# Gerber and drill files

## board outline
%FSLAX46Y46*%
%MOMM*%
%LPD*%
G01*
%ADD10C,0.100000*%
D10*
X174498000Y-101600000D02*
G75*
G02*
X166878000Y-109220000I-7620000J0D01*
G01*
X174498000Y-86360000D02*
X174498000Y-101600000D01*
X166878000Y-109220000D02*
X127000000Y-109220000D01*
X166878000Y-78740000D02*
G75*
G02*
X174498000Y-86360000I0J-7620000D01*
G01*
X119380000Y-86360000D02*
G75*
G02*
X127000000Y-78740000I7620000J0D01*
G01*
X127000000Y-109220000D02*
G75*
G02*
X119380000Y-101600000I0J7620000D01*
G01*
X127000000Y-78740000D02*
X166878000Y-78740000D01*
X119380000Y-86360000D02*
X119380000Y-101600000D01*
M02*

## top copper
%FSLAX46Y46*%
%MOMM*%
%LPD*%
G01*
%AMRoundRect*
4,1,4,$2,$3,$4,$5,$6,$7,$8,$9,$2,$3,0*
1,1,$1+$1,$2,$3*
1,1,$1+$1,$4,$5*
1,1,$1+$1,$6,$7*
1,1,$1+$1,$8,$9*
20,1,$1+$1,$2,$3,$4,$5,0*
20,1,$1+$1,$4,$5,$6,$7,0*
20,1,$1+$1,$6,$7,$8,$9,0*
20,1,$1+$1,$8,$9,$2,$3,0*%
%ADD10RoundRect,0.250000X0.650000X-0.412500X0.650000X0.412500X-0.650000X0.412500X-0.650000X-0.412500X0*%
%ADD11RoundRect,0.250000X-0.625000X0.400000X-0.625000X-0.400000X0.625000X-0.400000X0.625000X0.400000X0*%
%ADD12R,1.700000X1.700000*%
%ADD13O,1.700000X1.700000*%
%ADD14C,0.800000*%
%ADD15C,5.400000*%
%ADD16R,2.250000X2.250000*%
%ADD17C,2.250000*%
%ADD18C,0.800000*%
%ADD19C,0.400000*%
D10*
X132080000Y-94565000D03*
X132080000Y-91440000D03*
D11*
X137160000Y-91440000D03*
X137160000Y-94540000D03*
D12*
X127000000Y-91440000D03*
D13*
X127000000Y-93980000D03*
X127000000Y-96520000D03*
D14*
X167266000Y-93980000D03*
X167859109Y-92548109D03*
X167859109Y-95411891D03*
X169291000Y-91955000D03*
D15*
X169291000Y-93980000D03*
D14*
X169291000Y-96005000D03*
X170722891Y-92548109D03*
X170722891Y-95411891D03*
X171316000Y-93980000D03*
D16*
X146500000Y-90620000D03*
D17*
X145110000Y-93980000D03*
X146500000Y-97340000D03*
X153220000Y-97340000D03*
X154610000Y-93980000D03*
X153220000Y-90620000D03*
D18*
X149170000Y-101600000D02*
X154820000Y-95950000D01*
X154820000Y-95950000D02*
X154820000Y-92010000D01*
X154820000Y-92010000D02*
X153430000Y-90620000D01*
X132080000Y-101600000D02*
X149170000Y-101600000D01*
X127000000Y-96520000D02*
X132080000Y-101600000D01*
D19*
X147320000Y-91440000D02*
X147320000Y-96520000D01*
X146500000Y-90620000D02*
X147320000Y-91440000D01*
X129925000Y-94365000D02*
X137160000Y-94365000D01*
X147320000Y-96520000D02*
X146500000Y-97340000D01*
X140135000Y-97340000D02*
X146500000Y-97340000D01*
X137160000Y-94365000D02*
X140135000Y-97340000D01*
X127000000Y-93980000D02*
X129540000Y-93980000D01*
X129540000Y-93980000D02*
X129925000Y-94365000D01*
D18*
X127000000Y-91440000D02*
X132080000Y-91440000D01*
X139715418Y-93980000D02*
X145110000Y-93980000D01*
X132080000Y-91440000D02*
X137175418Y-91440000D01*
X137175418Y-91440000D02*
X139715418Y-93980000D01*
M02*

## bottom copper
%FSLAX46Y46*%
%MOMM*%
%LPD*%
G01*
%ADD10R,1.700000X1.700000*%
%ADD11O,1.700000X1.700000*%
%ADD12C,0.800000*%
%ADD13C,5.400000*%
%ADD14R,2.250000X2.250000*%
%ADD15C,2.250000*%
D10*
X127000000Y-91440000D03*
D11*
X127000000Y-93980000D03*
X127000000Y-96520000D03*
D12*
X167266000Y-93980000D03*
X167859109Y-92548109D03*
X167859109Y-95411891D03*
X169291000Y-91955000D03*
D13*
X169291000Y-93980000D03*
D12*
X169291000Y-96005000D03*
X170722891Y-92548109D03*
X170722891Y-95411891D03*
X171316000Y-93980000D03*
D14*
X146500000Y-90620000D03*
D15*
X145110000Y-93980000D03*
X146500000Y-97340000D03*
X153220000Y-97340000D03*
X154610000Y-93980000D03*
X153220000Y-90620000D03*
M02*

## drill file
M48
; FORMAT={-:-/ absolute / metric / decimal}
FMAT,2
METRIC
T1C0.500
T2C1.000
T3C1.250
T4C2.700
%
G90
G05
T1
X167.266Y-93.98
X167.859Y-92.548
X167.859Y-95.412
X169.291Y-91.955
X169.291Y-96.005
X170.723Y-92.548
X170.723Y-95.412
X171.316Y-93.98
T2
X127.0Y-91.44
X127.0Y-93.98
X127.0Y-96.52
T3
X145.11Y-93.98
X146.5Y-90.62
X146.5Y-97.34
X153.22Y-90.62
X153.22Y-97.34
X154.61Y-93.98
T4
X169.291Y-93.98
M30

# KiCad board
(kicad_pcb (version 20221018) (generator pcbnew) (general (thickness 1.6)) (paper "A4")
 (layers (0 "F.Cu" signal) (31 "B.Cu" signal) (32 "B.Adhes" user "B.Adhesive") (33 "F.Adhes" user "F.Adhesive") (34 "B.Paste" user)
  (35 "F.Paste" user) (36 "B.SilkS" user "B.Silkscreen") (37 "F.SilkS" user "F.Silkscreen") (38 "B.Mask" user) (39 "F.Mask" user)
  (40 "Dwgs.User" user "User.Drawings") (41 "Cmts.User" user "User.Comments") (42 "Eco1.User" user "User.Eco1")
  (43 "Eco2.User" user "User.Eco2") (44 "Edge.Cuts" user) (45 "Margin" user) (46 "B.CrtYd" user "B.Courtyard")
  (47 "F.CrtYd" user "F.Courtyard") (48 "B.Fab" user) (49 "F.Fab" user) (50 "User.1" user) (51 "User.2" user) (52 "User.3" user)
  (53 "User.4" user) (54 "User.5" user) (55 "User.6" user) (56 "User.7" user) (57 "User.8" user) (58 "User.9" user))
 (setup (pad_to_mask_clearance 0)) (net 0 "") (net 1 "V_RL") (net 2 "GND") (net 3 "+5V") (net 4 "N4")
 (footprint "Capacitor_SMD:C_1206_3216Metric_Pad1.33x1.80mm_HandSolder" (layer "F.Cu") (at 132.08 93.0025 90)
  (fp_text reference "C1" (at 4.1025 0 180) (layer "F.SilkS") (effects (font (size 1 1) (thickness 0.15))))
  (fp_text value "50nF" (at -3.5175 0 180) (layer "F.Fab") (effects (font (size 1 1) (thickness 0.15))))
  (pad "1" smd roundrect (at -1.5625 0 90) (size 1.325 1.8) (layers "F.Cu" "F.Paste" "F.Mask") (roundrect_rratio 0.1886792453)
   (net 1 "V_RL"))
  (pad "2" smd roundrect (at 1.5625 0 90) (size 1.325 1.8) (layers "F.Cu" "F.Paste" "F.Mask") (roundrect_rratio 0.1886792453) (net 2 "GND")))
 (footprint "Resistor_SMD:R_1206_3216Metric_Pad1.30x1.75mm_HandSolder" (layer "F.Cu") (at 137.16 92.99 -90)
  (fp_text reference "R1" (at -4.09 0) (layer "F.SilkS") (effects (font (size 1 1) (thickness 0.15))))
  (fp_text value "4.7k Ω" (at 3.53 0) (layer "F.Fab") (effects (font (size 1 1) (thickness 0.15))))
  (pad "1" smd roundrect (at -1.55 0 270) (size 1.3 1.75) (layers "F.Cu" "F.Paste" "F.Mask") (roundrect_rratio 0.1923076923) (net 2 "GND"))
  (pad "2" smd roundrect (at 1.55 0 270) (size 1.3 1.75) (layers "F.Cu" "F.Paste" "F.Mask") (roundrect_rratio 0.1923076923) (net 1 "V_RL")))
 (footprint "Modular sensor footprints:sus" (layer "F.Cu") (at 149.86 93.98)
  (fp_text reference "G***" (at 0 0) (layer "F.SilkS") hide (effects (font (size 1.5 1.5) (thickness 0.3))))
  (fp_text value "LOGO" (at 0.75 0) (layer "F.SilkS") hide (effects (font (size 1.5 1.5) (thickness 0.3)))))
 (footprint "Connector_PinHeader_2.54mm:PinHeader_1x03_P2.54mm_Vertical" (layer "F.Cu") (at 127 91.44)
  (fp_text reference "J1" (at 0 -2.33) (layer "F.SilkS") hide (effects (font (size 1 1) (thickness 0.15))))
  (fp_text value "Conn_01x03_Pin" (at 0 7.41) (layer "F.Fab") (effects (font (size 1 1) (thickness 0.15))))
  (pad "1" thru_hole rect (at 0 0) (size 1.7 1.7) (drill 1) (layers "*.Cu" "*.Mask") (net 2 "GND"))
  (pad "2" thru_hole oval (at 0 2.54) (size 1.7 1.7) (drill 1) (layers "*.Cu" "*.Mask") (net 1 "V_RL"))
  (pad "3" thru_hole oval (at 0 5.08) (size 1.7 1.7) (drill 1) (layers "*.Cu" "*.Mask") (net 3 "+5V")))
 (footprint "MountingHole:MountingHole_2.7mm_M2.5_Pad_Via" (layer "F.Cu") (at 169.291 93.98)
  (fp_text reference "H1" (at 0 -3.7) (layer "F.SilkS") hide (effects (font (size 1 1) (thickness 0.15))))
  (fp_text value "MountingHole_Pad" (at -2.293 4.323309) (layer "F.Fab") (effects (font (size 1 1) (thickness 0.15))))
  (pad "1" thru_hole circle (at -2.025 0) (size 0.8 0.8) (drill 0.5) (layers "*.Cu" "*.Mask") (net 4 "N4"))
  (pad "1" thru_hole circle (at -1.431891 -1.431891) (size 0.8 0.8) (drill 0.5) (layers "*.Cu" "*.Mask") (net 4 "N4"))
  (pad "1" thru_hole circle (at -1.431891 1.431891) (size 0.8 0.8) (drill 0.5) (layers "*.Cu" "*.Mask") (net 4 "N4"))
  (pad "1" thru_hole circle (at 0 -2.025) (size 0.8 0.8) (drill 0.5) (layers "*.Cu" "*.Mask") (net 4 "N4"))
  (pad "1" thru_hole circle (at 0 0) (size 5.4 5.4) (drill 2.7) (layers "*.Cu" "*.Mask") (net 4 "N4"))
  (pad "1" thru_hole circle (at 0 2.025) (size 0.8 0.8) (drill 0.5) (layers "*.Cu" "*.Mask") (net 4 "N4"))
  (pad "1" thru_hole circle (at 1.431891 -1.431891) (size 0.8 0.8) (drill 0.5) (layers "*.Cu" "*.Mask") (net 4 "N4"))
  (pad "1" thru_hole circle (at 1.431891 1.431891) (size 0.8 0.8) (drill 0.5) (layers "*.Cu" "*.Mask") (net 4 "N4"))
  (pad "1" thru_hole circle (at 2.025 0) (size 0.8 0.8) (drill 0.5) (layers "*.Cu" "*.Mask") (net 4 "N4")))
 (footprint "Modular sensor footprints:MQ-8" (layer "F.Cu") (at 146.5 90.62)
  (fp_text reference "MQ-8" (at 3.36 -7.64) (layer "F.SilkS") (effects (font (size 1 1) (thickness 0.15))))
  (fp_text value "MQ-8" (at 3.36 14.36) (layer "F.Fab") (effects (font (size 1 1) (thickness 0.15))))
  (pad "1" thru_hole rect (at 0 0) (size 2.25 2.25) (drill 1.25) (layers "*.Cu" "*.Mask") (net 1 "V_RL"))
  (pad "2" thru_hole circle (at -1.39 3.36) (size 2.25 2.25) (drill 1.25) (layers "*.Cu" "*.Mask") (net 2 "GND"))
  (pad "3" thru_hole circle (at 0 6.72 90) (size 2.25 2.25) (drill 1.25) (layers "*.Cu" "*.Mask") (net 1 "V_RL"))
  (pad "4" thru_hole circle (at 6.72 6.72 180) (size 2.25 2.25) (drill 1.25) (layers "*.Cu" "*.Mask") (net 3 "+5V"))
  (pad "5" thru_hole circle (at 8.11 3.36) (size 2.25 2.25) (drill 1.25) (layers "*.Cu" "*.Mask") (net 3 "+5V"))
  (pad "6" thru_hole circle (at 6.72 0 270) (size 2.25 2.25) (drill 1.25) (layers "*.Cu" "*.Mask") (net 3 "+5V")))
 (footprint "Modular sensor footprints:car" (layer "B.Cu") (at 157.528157 83.771147 180)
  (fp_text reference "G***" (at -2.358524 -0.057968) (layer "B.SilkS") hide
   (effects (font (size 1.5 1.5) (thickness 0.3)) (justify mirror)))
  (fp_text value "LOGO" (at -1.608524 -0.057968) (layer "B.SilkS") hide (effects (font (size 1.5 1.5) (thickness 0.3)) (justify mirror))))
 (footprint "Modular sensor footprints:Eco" (layer "B.Cu") (at 160.02 83.82 180)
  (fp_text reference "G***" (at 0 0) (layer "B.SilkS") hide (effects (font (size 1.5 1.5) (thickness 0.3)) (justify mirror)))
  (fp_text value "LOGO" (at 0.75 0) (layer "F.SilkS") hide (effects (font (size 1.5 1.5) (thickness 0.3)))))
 (gr_arc (start 174.498 101.6) (mid 172.266154 106.988154) (end 166.878 109.22) (stroke (width 0.1) (type default)) (layer "Edge.Cuts"))
 (gr_line (start 174.498 86.36) (end 174.498 101.6) (stroke (width 0.1) (type default)) (layer "Edge.Cuts"))
 (gr_line (start 166.878 109.22) (end 127 109.22) (stroke (width 0.1) (type default)) (layer "Edge.Cuts"))
 (gr_arc (start 166.878 78.74) (mid 172.266154 80.971846) (end 174.498 86.36) (stroke (width 0.1) (type default)) (layer "Edge.Cuts"))
 (gr_arc (start 119.38 86.36) (mid 121.611846 80.971846) (end 127 78.74) (stroke (width 0.1) (type default)) (layer "Edge.Cuts"))
 (gr_arc (start 127 109.22) (mid 121.611846 106.988154) (end 119.38 101.6) (stroke (width 0.1) (type default)) (layer "Edge.Cuts"))
 (gr_line (start 127 78.74) (end 166.878 78.74) (stroke (width 0.1) (type default)) (layer "Edge.Cuts"))
 (gr_line (start 119.38 86.36) (end 119.38 101.6) (stroke (width 0.1) (type default)) (layer "Edge.Cuts"))
 (segment (start 149.17 101.6) (end 154.82 95.95) (width 0.8) (layer "F.Cu") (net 3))
 (segment (start 154.82 95.95) (end 154.82 92.01) (width 0.8) (layer "F.Cu") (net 3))
 (segment (start 154.82 92.01) (end 153.43 90.62) (width 0.8) (layer "F.Cu") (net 3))
 (segment (start 132.08 101.6) (end 149.17 101.6) (width 0.8) (layer "F.Cu") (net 3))
 (segment (start 127 96.52) (end 132.08 101.6) (width 0.8) (layer "F.Cu") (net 3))
 (segment (start 147.32 91.44) (end 147.32 96.52) (width 0.4) (layer "F.Cu") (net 1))
 (segment (start 146.5 90.62) (end 147.32 91.44) (width 0.4) (layer "F.Cu") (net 1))
 (segment (start 129.925 94.365) (end 137.16 94.365) (width 0.4) (layer "F.Cu") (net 1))
 (segment (start 147.32 96.52) (end 146.5 97.34) (width 0.4) (layer "F.Cu") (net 1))
 (segment (start 140.135 97.34) (end 146.5 97.34) (width 0.4) (layer "F.Cu") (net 1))
 (segment (start 137.16 94.365) (end 140.135 97.34) (width 0.4) (layer "F.Cu") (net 1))
 (segment (start 127 93.98) (end 129.54 93.98) (width 0.4) (layer "F.Cu") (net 1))
 (segment (start 129.54 93.98) (end 129.925 94.365) (width 0.4) (layer "F.Cu") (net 1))
 (segment (start 127 91.44) (end 132.08 91.44) (width 0.8) (layer "F.Cu") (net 2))
 (segment (start 139.715418 93.98) (end 145.11 93.98) (width 0.8) (layer "F.Cu") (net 2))
 (segment (start 132.08 91.44) (end 137.175418 91.44) (width 0.8) (layer "F.Cu") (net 2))
 (segment (start 137.175418 91.44) (end 139.715418 93.98) (width 0.8) (layer "F.Cu") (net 2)))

